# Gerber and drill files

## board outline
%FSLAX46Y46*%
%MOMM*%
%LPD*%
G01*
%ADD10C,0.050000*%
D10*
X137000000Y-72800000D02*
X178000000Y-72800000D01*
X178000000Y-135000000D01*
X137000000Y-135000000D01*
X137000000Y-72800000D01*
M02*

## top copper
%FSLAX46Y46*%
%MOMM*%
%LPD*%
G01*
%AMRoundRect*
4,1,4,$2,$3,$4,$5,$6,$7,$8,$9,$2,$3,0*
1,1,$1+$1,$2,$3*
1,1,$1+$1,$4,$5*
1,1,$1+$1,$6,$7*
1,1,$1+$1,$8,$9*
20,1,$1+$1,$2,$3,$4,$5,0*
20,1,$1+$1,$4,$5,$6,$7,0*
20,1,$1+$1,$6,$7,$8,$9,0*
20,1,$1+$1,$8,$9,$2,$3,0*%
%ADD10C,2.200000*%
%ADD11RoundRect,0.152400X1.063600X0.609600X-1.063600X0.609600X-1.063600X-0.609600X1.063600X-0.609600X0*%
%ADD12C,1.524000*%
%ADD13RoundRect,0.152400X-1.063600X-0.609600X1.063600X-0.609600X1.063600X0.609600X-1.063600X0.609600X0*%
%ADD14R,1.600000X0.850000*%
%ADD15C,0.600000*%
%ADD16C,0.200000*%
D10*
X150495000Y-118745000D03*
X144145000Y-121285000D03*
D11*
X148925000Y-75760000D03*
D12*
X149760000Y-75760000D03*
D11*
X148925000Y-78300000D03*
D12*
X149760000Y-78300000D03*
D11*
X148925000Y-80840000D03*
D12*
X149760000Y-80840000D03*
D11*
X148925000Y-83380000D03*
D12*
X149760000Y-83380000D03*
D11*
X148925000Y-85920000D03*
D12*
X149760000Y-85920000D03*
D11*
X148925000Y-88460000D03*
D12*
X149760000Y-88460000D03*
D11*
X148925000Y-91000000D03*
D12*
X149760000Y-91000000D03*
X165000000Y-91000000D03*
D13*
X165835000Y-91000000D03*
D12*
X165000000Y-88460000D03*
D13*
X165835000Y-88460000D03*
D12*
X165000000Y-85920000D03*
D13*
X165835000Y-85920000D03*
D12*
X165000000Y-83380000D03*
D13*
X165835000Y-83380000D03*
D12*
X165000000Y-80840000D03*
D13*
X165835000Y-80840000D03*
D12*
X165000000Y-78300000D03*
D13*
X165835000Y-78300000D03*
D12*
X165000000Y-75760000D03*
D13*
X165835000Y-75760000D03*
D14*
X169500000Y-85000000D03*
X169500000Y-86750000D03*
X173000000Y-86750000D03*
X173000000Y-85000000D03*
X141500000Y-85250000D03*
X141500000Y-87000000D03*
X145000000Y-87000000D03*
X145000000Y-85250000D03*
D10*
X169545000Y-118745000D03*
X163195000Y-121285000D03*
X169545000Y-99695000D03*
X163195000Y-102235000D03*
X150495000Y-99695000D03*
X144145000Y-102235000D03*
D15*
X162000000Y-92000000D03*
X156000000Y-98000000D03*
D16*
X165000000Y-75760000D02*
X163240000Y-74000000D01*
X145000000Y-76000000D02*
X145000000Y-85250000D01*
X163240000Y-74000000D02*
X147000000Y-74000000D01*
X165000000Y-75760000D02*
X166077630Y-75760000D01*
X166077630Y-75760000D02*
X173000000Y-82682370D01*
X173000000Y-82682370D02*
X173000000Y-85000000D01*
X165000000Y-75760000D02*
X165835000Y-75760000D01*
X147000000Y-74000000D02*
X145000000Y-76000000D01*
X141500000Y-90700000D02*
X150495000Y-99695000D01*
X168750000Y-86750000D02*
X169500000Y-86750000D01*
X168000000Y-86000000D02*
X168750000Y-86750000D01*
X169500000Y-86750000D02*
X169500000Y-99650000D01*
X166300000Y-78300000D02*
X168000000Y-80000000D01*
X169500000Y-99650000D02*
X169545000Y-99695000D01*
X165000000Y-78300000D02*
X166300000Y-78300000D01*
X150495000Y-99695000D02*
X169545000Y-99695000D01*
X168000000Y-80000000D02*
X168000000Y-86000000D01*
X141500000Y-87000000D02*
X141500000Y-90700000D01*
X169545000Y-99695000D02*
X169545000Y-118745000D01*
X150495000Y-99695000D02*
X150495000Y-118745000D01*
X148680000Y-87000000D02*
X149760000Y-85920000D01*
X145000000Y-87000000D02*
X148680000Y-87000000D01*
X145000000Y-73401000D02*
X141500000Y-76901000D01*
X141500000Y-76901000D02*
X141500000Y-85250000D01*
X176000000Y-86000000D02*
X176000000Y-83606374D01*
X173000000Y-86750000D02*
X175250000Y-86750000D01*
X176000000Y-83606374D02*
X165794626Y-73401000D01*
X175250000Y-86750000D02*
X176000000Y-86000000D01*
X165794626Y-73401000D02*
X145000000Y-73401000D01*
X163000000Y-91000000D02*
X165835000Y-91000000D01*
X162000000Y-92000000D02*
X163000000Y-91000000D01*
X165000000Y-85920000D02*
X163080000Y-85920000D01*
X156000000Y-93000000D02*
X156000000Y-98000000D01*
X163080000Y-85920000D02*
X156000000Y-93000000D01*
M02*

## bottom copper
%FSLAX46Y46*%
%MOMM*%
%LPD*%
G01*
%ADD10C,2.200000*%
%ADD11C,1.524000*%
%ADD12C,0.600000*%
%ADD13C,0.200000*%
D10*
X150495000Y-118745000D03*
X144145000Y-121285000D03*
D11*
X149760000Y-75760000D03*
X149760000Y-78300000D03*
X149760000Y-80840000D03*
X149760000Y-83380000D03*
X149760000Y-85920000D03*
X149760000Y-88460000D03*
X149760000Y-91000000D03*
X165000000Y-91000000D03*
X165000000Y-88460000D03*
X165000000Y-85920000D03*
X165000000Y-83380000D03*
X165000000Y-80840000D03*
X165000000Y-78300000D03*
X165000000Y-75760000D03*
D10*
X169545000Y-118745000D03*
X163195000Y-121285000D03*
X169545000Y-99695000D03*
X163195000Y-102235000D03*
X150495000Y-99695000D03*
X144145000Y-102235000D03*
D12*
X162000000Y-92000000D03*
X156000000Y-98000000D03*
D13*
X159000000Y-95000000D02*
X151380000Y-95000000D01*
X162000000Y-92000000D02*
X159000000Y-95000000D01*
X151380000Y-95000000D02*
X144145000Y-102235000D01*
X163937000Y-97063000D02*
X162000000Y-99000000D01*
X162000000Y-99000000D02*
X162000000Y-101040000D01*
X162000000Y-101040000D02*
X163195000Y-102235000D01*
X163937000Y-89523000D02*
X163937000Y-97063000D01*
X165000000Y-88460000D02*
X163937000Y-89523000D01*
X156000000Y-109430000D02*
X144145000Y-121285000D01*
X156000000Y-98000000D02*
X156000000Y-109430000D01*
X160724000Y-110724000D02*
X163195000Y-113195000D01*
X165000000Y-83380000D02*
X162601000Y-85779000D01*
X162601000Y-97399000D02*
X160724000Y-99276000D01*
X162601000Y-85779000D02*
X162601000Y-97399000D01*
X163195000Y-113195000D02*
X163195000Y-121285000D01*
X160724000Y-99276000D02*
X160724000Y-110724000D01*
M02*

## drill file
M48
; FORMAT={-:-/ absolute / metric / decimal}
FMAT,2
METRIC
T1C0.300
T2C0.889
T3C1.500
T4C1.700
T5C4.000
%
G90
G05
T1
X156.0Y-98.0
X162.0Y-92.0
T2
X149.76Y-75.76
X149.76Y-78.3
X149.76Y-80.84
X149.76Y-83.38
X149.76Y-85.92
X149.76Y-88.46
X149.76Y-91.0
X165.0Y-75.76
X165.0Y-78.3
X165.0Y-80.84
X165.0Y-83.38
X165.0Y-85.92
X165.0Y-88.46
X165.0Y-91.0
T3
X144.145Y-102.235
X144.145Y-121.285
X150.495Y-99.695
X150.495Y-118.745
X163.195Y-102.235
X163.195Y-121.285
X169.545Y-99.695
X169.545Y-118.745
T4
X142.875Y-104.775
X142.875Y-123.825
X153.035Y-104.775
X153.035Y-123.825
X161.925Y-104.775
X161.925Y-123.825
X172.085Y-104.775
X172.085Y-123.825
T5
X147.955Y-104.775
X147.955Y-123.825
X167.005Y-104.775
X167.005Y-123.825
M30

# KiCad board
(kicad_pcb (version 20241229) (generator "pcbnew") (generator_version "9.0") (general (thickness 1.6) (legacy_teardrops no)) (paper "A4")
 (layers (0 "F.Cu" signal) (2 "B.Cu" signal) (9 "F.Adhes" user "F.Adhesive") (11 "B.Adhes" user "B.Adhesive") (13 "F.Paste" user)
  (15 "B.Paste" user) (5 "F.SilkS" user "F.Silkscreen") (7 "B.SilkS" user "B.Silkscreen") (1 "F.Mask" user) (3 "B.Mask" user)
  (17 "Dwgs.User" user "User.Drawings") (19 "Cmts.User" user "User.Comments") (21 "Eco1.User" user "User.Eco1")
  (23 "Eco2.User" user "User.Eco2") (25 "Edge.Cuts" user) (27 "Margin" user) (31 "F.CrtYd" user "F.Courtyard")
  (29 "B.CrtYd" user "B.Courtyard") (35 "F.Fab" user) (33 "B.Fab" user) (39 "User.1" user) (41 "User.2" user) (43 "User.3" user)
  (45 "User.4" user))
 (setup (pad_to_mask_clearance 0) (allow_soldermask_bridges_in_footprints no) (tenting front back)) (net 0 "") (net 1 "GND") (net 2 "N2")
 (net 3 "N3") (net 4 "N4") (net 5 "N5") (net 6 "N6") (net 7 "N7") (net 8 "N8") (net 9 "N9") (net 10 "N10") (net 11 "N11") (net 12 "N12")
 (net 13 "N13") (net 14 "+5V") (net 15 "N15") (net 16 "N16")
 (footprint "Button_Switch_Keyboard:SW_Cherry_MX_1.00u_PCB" (layer "F.Cu") (at 150.495 118.745)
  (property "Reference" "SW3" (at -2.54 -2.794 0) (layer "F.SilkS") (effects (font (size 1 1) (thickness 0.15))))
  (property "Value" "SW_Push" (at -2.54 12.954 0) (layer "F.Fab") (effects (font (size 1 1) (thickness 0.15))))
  (pad "" np_thru_hole circle (at -7.62 5.08) (size 1.7 1.7) (drill 1.7) (layers "*.Cu" "*.Mask"))
  (pad "" np_thru_hole circle (at -2.54 5.08) (size 4 4) (drill 4) (layers "*.Cu" "*.Mask"))
  (pad "" np_thru_hole circle (at 2.54 5.08) (size 1.7 1.7) (drill 1.7) (layers "*.Cu" "*.Mask"))
  (pad "1" thru_hole circle (at 0 0) (size 2.2 2.2) (drill 1.5) (layers "*.Cu" "*.Mask") (remove_unused_layers no) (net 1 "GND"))
  (pad "2" thru_hole circle (at -6.35 2.54) (size 2.2 2.2) (drill 1.5) (layers "*.Cu" "*.Mask") (remove_unused_layers no) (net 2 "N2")))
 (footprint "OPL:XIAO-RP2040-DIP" (layer "F.Cu") (at 157.38 83.38)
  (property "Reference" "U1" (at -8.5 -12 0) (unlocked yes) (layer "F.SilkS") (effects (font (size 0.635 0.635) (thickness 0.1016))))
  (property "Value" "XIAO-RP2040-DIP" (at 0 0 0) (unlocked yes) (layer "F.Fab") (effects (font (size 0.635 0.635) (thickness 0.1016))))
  (pad "1" smd roundrect (at -8.455 -7.62 180) (size 2.432 1.524) (layers "F.Cu" "F.Mask") (roundrect_rratio 0.1) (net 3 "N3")
   (thermal_bridge_angle 45))
  (pad "1" thru_hole circle (at -7.62 -7.62 180) (size 1.524 1.524) (drill 0.889) (layers "*.Cu" "*.Mask") (remove_unused_layers no)
   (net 3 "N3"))
  (pad "2" smd roundrect (at -8.455 -5.08 180) (size 2.432 1.524) (layers "F.Cu" "F.Mask") (roundrect_rratio 0.1) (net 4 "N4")
   (thermal_bridge_angle 45))
  (pad "2" thru_hole circle (at -7.62 -5.08 180) (size 1.524 1.524) (drill 0.889) (layers "*.Cu" "*.Mask") (remove_unused_layers no)
   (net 4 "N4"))
  (pad "3" smd roundrect (at -8.455 -2.54 180) (size 2.432 1.524) (layers "F.Cu" "F.Mask") (roundrect_rratio 0.1) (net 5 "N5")
   (thermal_bridge_angle 45))
  (pad "3" thru_hole circle (at -7.62 -2.54 180) (size 1.524 1.524) (drill 0.889) (layers "*.Cu" "*.Mask") (remove_unused_layers no)
   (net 5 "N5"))
  (pad "4" smd roundrect (at -8.455 0 180) (size 2.432 1.524) (layers "F.Cu" "F.Mask") (roundrect_rratio 0.1) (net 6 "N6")
   (thermal_bridge_angle 45))
  (pad "4" thru_hole circle (at -7.62 0 180) (size 1.524 1.524) (drill 0.889) (layers "*.Cu" "*.Mask") (remove_unused_layers no)
   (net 6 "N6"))
  (pad "5" smd roundrect (at -8.455 2.54 180) (size 2.432 1.524) (layers "F.Cu" "F.Mask") (roundrect_rratio 0.1) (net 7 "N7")
   (thermal_bridge_angle 45))
  (pad "5" thru_hole circle (at -7.62 2.54 180) (size 1.524 1.524) (drill 0.889) (layers "*.Cu" "*.Mask") (remove_unused_layers no)
   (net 7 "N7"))
  (pad "6" smd roundrect (at -8.455 5.08 180) (size 2.432 1.524) (layers "F.Cu" "F.Mask") (roundrect_rratio 0.1) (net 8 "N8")
   (thermal_bridge_angle 45))
  (pad "6" thru_hole circle (at -7.62 5.08 180) (size 1.524 1.524) (drill 0.889) (layers "*.Cu" "*.Mask") (remove_unused_layers no)
   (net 8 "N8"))
  (pad "7" smd roundrect (at -8.455 7.62 180) (size 2.432 1.524) (layers "F.Cu" "F.Mask") (roundrect_rratio 0.1) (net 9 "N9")
   (thermal_bridge_angle 45))
  (pad "7" thru_hole circle (at -7.62 7.62 180) (size 1.524 1.524) (drill 0.889) (layers "*.Cu" "*.Mask") (remove_unused_layers no)
   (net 9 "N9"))
  (pad "8" thru_hole circle (at 7.62 7.62) (size 1.524 1.524) (drill 0.889) (layers "*.Cu" "*.Mask") (remove_unused_layers no)
   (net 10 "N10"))
  (pad "8" smd roundrect (at 8.455 7.62) (size 2.432 1.524) (layers "F.Cu" "F.Mask") (roundrect_rratio 0.1) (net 10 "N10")
   (thermal_bridge_angle 45))
  (pad "9" thru_hole circle (at 7.62 5.08) (size 1.524 1.524) (drill 0.889) (layers "*.Cu" "*.Mask") (remove_unused_layers no)
   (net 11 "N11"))
  (pad "9" smd roundrect (at 8.455 5.08) (size 2.432 1.524) (layers "F.Cu" "F.Mask") (roundrect_rratio 0.1) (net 11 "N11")
   (thermal_bridge_angle 45))
  (pad "10" thru_hole circle (at 7.62 2.54) (size 1.524 1.524) (drill 0.889) (layers "*.Cu" "*.Mask") (remove_unused_layers no) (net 2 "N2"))
  (pad "10" smd roundrect (at 8.455 2.54) (size 2.432 1.524) (layers "F.Cu" "F.Mask") (roundrect_rratio 0.1) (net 2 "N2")
   (thermal_bridge_angle 45))
  (pad "11" thru_hole circle (at 7.62 0) (size 1.524 1.524) (drill 0.889) (layers "*.Cu" "*.Mask") (remove_unused_layers no) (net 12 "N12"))
  (pad "11" smd roundrect (at 8.455 0) (size 2.432 1.524) (layers "F.Cu" "F.Mask") (roundrect_rratio 0.1) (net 12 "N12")
   (thermal_bridge_angle 45))
  (pad "12" thru_hole circle (at 7.62 -2.54) (size 1.524 1.524) (drill 0.889) (layers "*.Cu" "*.Mask") (remove_unused_layers no)
   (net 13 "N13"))
  (pad "12" smd roundrect (at 8.455 -2.54) (size 2.432 1.524) (layers "F.Cu" "F.Mask") (roundrect_rratio 0.1) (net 13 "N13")
   (thermal_bridge_angle 45))
  (pad "13" thru_hole circle (at 7.62 -5.08) (size 1.524 1.524) (drill 0.889) (layers "*.Cu" "*.Mask") (remove_unused_layers no)
   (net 1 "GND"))
  (pad "13" smd roundrect (at 8.455 -5.08) (size 2.432 1.524) (layers "F.Cu" "F.Mask") (roundrect_rratio 0.1) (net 1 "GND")
   (thermal_bridge_angle 45))
  (pad "14" thru_hole circle (at 7.62 -7.62) (size 1.524 1.524) (drill 0.889) (layers "*.Cu" "*.Mask") (remove_unused_layers no)
   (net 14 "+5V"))
  (pad "14" smd roundrect (at 8.455 -7.62) (size 2.432 1.524) (layers "F.Cu" "F.Mask") (roundrect_rratio 0.1) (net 14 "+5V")
   (thermal_bridge_angle 45)))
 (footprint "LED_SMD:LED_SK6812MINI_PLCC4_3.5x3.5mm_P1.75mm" (layer "F.Cu") (at 171.25 85.875)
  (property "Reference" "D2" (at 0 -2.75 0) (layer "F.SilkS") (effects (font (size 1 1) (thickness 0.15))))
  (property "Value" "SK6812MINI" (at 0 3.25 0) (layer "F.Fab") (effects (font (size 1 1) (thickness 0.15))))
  (pad "1" smd rect (at -1.75 -0.875) (size 1.6 0.85) (layers "F.Cu" "F.Mask" "F.Paste") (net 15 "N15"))
  (pad "2" smd rect (at -1.75 0.875) (size 1.6 0.85) (layers "F.Cu" "F.Mask" "F.Paste") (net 1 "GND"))
  (pad "3" smd rect (at 1.75 0.875) (size 1.6 0.85) (layers "F.Cu" "F.Mask" "F.Paste") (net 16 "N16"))
  (pad "4" smd rect (at 1.75 -0.875) (size 1.6 0.85) (layers "F.Cu" "F.Mask" "F.Paste") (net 14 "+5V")))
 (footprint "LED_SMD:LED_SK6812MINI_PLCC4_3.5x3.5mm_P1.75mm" (layer "F.Cu") (at 143.25 86.125)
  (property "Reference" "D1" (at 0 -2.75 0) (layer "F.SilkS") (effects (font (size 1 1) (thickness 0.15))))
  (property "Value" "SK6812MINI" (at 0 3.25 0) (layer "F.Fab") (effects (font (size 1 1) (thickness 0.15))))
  (pad "1" smd rect (at -1.75 -0.875) (size 1.6 0.85) (layers "F.Cu" "F.Mask" "F.Paste") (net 16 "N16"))
  (pad "2" smd rect (at -1.75 0.875) (size 1.6 0.85) (layers "F.Cu" "F.Mask" "F.Paste") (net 1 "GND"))
  (pad "3" smd rect (at 1.75 0.875) (size 1.6 0.85) (layers "F.Cu" "F.Mask" "F.Paste") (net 7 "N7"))
  (pad "4" smd rect (at 1.75 -0.875) (size 1.6 0.85) (layers "F.Cu" "F.Mask" "F.Paste") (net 14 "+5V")))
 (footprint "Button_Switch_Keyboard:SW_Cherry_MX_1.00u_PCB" (layer "F.Cu") (at 169.545 118.745)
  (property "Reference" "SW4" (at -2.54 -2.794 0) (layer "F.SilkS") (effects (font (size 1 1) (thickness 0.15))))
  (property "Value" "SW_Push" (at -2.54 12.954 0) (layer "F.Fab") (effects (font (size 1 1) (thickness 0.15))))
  (pad "" np_thru_hole circle (at -7.62 5.08) (size 1.7 1.7) (drill 1.7) (layers "*.Cu" "*.Mask"))
  (pad "" np_thru_hole circle (at -2.54 5.08) (size 4 4) (drill 4) (layers "*.Cu" "*.Mask"))
  (pad "" np_thru_hole circle (at 2.54 5.08) (size 1.7 1.7) (drill 1.7) (layers "*.Cu" "*.Mask"))
  (pad "1" thru_hole circle (at 0 0) (size 2.2 2.2) (drill 1.5) (layers "*.Cu" "*.Mask") (remove_unused_layers no) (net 1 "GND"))
  (pad "2" thru_hole circle (at -6.35 2.54) (size 2.2 2.2) (drill 1.5) (layers "*.Cu" "*.Mask") (remove_unused_layers no) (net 12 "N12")))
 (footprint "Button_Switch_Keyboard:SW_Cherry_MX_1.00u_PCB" (layer "F.Cu") (at 169.545 99.695)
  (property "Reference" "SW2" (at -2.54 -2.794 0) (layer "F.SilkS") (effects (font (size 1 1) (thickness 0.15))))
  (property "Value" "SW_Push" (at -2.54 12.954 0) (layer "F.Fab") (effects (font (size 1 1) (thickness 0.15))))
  (pad "" np_thru_hole circle (at -7.62 5.08) (size 1.7 1.7) (drill 1.7) (layers "*.Cu" "*.Mask"))
  (pad "" np_thru_hole circle (at -2.54 5.08) (size 4 4) (drill 4) (layers "*.Cu" "*.Mask"))
  (pad "" np_thru_hole circle (at 2.54 5.08) (size 1.7 1.7) (drill 1.7) (layers "*.Cu" "*.Mask"))
  (pad "1" thru_hole circle (at 0 0) (size 2.2 2.2) (drill 1.5) (layers "*.Cu" "*.Mask") (remove_unused_layers no) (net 1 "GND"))
  (pad "2" thru_hole circle (at -6.35 2.54) (size 2.2 2.2) (drill 1.5) (layers "*.Cu" "*.Mask") (remove_unused_layers no) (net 11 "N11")))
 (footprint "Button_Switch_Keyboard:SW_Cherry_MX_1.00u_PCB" (layer "F.Cu") (at 150.495 99.695)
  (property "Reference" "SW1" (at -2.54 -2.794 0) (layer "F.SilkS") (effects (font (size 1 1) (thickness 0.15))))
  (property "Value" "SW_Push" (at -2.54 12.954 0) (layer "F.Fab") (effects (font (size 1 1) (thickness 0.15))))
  (pad "" np_thru_hole circle (at -7.62 5.08) (size 1.7 1.7) (drill 1.7) (layers "*.Cu" "*.Mask"))
  (pad "" np_thru_hole circle (at -2.54 5.08) (size 4 4) (drill 4) (layers "*.Cu" "*.Mask"))
  (pad "" np_thru_hole circle (at 2.54 5.08) (size 1.7 1.7) (drill 1.7) (layers "*.Cu" "*.Mask"))
  (pad "1" thru_hole circle (at 0 0) (size 2.2 2.2) (drill 1.5) (layers "*.Cu" "*.Mask") (remove_unused_layers no) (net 1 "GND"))
  (pad "2" thru_hole circle (at -6.35 2.54) (size 2.2 2.2) (drill 1.5) (layers "*.Cu" "*.Mask") (remove_unused_layers no) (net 10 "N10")))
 (gr_rect (start 137 72.8) (end 178 135) (stroke (width 0.05) (type default)) (fill no) (layer "Edge.Cuts"))
 (segment (start 165 75.76) (end 163.24 74) (width 0.2) (layer "F.Cu") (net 14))
 (segment (start 145 76) (end 145 85.25) (width 0.2) (layer "F.Cu") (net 14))
 (segment (start 163.24 74) (end 147 74) (width 0.2) (layer "F.Cu") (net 14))
 (segment (start 165 75.76) (end 166.07763 75.76) (width 0.2) (layer "F.Cu") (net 14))
 (segment (start 166.07763 75.76) (end 173 82.68237) (width 0.2) (layer "F.Cu") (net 14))
 (segment (start 173 82.68237) (end 173 85) (width 0.2) (layer "F.Cu") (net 14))
 (segment (start 165 75.76) (end 165.835 75.76) (width 0.2) (layer "F.Cu") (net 14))
 (segment (start 147 74) (end 145 76) (width 0.2) (layer "F.Cu") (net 14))
 (segment (start 141.5 90.7) (end 150.495 99.695) (width 0.2) (layer "F.Cu") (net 1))
 (segment (start 168.75 86.75) (end 169.5 86.75) (width 0.2) (layer "F.Cu") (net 1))
 (segment (start 168 86) (end 168.75 86.75) (width 0.2) (layer "F.Cu") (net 1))
 (segment (start 169.5 86.75) (end 169.5 99.65) (width 0.2) (layer "F.Cu") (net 1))
 (segment (start 166.3 78.3) (end 168 80) (width 0.2) (layer "F.Cu") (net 1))
 (segment (start 169.5 99.65) (end 169.545 99.695) (width 0.2) (layer "F.Cu") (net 1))
 (segment (start 165 78.3) (end 166.3 78.3) (width 0.2) (layer "F.Cu") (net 1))
 (segment (start 150.495 99.695) (end 169.545 99.695) (width 0.2) (layer "F.Cu") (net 1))
 (segment (start 168 80) (end 168 86) (width 0.2) (layer "F.Cu") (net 1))
 (segment (start 141.5 87) (end 141.5 90.7) (width 0.2) (layer "F.Cu") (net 1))
 (segment (start 169.545 99.695) (end 169.545 118.745) (width 0.2) (layer "F.Cu") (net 1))
 (segment (start 150.495 99.695) (end 150.495 118.745) (width 0.2) (layer "F.Cu") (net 1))
 (segment (start 148.68 87) (end 149.76 85.92) (width 0.2) (layer "F.Cu") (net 7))
 (segment (start 145 87) (end 148.68 87) (width 0.2) (layer "F.Cu") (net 7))
 (segment (start 145 73.401) (end 141.5 76.901) (width 0.2) (layer "F.Cu") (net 16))
 (segment (start 141.5 76.901) (end 141.5 85.25) (width 0.2) (layer "F.Cu") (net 16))
 (segment (start 176 86) (end 176 83.606374) (width 0.2) (layer "F.Cu") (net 16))
 (segment (start 173 86.75) (end 175.25 86.75) (width 0.2) (layer "F.Cu") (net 16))
 (segment (start 176 83.606374) (end 165.794626 73.401) (width 0.2) (layer "F.Cu") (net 16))
 (segment (start 175.25 86.75) (end 176 86) (width 0.2) (layer "F.Cu") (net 16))
 (segment (start 165.794626 73.401) (end 145 73.401) (width 0.2) (layer "F.Cu") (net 16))
 (segment (start 163 91) (end 165.835 91) (width 0.2) (layer "F.Cu") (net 10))
 (segment (start 162 92) (end 163 91) (width 0.2) (layer "F.Cu") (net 10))
 (via (at 162 92) (size 0.6) (drill 0.3) (layers "F.Cu" "B.Cu") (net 10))
 (segment (start 159 95) (end 151.38 95) (width 0.2) (layer "B.Cu") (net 10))
 (segment (start 162 92) (end 159 95) (width 0.2) (layer "B.Cu") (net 10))
 (segment (start 151.38 95) (end 144.145 102.235) (width 0.2) (layer "B.Cu") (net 10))
 (segment (start 163.937 97.063) (end 162 99) (width 0.2) (layer "B.Cu") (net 11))
 (segment (start 162 99) (end 162 101.04) (width 0.2) (layer "B.Cu") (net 11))
 (segment (start 162 101.04) (end 163.195 102.235) (width 0.2) (layer "B.Cu") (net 11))
 (segment (start 163.937 89.523) (end 163.937 97.063) (width 0.2) (layer "B.Cu") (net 11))
 (segment (start 165 88.46) (end 163.937 89.523) (width 0.2) (layer "B.Cu") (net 11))
 (segment (start 165 85.92) (end 163.08 85.92) (width 0.2) (layer "F.Cu") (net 2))
 (segment (start 156 93) (end 156 98) (width 0.2) (layer "F.Cu") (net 2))
 (segment (start 163.08 85.92) (end 156 93) (width 0.2) (layer "F.Cu") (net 2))
 (via (at 156 98) (size 0.6) (drill 0.3) (layers "F.Cu" "B.Cu") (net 2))
 (segment (start 156 109.43) (end 144.145 121.285) (width 0.2) (layer "B.Cu") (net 2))
 (segment (start 156 98) (end 156 109.43) (width 0.2) (layer "B.Cu") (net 2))
 (segment (start 160.724 110.724) (end 163.195 113.195) (width 0.2) (layer "B.Cu") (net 12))
 (segment (start 165 83.38) (end 162.601 85.779) (width 0.2) (layer "B.Cu") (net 12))
 (segment (start 162.601 97.399) (end 160.724 99.276) (width 0.2) (layer "B.Cu") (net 12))
 (segment (start 162.601 85.779) (end 162.601 97.399) (width 0.2) (layer "B.Cu") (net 12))
 (segment (start 163.195 113.195) (end 163.195 121.285) (width 0.2) (layer "B.Cu") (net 12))
 (segment (start 160.724 99.276) (end 160.724 110.724) (width 0.2) (layer "B.Cu") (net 12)))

